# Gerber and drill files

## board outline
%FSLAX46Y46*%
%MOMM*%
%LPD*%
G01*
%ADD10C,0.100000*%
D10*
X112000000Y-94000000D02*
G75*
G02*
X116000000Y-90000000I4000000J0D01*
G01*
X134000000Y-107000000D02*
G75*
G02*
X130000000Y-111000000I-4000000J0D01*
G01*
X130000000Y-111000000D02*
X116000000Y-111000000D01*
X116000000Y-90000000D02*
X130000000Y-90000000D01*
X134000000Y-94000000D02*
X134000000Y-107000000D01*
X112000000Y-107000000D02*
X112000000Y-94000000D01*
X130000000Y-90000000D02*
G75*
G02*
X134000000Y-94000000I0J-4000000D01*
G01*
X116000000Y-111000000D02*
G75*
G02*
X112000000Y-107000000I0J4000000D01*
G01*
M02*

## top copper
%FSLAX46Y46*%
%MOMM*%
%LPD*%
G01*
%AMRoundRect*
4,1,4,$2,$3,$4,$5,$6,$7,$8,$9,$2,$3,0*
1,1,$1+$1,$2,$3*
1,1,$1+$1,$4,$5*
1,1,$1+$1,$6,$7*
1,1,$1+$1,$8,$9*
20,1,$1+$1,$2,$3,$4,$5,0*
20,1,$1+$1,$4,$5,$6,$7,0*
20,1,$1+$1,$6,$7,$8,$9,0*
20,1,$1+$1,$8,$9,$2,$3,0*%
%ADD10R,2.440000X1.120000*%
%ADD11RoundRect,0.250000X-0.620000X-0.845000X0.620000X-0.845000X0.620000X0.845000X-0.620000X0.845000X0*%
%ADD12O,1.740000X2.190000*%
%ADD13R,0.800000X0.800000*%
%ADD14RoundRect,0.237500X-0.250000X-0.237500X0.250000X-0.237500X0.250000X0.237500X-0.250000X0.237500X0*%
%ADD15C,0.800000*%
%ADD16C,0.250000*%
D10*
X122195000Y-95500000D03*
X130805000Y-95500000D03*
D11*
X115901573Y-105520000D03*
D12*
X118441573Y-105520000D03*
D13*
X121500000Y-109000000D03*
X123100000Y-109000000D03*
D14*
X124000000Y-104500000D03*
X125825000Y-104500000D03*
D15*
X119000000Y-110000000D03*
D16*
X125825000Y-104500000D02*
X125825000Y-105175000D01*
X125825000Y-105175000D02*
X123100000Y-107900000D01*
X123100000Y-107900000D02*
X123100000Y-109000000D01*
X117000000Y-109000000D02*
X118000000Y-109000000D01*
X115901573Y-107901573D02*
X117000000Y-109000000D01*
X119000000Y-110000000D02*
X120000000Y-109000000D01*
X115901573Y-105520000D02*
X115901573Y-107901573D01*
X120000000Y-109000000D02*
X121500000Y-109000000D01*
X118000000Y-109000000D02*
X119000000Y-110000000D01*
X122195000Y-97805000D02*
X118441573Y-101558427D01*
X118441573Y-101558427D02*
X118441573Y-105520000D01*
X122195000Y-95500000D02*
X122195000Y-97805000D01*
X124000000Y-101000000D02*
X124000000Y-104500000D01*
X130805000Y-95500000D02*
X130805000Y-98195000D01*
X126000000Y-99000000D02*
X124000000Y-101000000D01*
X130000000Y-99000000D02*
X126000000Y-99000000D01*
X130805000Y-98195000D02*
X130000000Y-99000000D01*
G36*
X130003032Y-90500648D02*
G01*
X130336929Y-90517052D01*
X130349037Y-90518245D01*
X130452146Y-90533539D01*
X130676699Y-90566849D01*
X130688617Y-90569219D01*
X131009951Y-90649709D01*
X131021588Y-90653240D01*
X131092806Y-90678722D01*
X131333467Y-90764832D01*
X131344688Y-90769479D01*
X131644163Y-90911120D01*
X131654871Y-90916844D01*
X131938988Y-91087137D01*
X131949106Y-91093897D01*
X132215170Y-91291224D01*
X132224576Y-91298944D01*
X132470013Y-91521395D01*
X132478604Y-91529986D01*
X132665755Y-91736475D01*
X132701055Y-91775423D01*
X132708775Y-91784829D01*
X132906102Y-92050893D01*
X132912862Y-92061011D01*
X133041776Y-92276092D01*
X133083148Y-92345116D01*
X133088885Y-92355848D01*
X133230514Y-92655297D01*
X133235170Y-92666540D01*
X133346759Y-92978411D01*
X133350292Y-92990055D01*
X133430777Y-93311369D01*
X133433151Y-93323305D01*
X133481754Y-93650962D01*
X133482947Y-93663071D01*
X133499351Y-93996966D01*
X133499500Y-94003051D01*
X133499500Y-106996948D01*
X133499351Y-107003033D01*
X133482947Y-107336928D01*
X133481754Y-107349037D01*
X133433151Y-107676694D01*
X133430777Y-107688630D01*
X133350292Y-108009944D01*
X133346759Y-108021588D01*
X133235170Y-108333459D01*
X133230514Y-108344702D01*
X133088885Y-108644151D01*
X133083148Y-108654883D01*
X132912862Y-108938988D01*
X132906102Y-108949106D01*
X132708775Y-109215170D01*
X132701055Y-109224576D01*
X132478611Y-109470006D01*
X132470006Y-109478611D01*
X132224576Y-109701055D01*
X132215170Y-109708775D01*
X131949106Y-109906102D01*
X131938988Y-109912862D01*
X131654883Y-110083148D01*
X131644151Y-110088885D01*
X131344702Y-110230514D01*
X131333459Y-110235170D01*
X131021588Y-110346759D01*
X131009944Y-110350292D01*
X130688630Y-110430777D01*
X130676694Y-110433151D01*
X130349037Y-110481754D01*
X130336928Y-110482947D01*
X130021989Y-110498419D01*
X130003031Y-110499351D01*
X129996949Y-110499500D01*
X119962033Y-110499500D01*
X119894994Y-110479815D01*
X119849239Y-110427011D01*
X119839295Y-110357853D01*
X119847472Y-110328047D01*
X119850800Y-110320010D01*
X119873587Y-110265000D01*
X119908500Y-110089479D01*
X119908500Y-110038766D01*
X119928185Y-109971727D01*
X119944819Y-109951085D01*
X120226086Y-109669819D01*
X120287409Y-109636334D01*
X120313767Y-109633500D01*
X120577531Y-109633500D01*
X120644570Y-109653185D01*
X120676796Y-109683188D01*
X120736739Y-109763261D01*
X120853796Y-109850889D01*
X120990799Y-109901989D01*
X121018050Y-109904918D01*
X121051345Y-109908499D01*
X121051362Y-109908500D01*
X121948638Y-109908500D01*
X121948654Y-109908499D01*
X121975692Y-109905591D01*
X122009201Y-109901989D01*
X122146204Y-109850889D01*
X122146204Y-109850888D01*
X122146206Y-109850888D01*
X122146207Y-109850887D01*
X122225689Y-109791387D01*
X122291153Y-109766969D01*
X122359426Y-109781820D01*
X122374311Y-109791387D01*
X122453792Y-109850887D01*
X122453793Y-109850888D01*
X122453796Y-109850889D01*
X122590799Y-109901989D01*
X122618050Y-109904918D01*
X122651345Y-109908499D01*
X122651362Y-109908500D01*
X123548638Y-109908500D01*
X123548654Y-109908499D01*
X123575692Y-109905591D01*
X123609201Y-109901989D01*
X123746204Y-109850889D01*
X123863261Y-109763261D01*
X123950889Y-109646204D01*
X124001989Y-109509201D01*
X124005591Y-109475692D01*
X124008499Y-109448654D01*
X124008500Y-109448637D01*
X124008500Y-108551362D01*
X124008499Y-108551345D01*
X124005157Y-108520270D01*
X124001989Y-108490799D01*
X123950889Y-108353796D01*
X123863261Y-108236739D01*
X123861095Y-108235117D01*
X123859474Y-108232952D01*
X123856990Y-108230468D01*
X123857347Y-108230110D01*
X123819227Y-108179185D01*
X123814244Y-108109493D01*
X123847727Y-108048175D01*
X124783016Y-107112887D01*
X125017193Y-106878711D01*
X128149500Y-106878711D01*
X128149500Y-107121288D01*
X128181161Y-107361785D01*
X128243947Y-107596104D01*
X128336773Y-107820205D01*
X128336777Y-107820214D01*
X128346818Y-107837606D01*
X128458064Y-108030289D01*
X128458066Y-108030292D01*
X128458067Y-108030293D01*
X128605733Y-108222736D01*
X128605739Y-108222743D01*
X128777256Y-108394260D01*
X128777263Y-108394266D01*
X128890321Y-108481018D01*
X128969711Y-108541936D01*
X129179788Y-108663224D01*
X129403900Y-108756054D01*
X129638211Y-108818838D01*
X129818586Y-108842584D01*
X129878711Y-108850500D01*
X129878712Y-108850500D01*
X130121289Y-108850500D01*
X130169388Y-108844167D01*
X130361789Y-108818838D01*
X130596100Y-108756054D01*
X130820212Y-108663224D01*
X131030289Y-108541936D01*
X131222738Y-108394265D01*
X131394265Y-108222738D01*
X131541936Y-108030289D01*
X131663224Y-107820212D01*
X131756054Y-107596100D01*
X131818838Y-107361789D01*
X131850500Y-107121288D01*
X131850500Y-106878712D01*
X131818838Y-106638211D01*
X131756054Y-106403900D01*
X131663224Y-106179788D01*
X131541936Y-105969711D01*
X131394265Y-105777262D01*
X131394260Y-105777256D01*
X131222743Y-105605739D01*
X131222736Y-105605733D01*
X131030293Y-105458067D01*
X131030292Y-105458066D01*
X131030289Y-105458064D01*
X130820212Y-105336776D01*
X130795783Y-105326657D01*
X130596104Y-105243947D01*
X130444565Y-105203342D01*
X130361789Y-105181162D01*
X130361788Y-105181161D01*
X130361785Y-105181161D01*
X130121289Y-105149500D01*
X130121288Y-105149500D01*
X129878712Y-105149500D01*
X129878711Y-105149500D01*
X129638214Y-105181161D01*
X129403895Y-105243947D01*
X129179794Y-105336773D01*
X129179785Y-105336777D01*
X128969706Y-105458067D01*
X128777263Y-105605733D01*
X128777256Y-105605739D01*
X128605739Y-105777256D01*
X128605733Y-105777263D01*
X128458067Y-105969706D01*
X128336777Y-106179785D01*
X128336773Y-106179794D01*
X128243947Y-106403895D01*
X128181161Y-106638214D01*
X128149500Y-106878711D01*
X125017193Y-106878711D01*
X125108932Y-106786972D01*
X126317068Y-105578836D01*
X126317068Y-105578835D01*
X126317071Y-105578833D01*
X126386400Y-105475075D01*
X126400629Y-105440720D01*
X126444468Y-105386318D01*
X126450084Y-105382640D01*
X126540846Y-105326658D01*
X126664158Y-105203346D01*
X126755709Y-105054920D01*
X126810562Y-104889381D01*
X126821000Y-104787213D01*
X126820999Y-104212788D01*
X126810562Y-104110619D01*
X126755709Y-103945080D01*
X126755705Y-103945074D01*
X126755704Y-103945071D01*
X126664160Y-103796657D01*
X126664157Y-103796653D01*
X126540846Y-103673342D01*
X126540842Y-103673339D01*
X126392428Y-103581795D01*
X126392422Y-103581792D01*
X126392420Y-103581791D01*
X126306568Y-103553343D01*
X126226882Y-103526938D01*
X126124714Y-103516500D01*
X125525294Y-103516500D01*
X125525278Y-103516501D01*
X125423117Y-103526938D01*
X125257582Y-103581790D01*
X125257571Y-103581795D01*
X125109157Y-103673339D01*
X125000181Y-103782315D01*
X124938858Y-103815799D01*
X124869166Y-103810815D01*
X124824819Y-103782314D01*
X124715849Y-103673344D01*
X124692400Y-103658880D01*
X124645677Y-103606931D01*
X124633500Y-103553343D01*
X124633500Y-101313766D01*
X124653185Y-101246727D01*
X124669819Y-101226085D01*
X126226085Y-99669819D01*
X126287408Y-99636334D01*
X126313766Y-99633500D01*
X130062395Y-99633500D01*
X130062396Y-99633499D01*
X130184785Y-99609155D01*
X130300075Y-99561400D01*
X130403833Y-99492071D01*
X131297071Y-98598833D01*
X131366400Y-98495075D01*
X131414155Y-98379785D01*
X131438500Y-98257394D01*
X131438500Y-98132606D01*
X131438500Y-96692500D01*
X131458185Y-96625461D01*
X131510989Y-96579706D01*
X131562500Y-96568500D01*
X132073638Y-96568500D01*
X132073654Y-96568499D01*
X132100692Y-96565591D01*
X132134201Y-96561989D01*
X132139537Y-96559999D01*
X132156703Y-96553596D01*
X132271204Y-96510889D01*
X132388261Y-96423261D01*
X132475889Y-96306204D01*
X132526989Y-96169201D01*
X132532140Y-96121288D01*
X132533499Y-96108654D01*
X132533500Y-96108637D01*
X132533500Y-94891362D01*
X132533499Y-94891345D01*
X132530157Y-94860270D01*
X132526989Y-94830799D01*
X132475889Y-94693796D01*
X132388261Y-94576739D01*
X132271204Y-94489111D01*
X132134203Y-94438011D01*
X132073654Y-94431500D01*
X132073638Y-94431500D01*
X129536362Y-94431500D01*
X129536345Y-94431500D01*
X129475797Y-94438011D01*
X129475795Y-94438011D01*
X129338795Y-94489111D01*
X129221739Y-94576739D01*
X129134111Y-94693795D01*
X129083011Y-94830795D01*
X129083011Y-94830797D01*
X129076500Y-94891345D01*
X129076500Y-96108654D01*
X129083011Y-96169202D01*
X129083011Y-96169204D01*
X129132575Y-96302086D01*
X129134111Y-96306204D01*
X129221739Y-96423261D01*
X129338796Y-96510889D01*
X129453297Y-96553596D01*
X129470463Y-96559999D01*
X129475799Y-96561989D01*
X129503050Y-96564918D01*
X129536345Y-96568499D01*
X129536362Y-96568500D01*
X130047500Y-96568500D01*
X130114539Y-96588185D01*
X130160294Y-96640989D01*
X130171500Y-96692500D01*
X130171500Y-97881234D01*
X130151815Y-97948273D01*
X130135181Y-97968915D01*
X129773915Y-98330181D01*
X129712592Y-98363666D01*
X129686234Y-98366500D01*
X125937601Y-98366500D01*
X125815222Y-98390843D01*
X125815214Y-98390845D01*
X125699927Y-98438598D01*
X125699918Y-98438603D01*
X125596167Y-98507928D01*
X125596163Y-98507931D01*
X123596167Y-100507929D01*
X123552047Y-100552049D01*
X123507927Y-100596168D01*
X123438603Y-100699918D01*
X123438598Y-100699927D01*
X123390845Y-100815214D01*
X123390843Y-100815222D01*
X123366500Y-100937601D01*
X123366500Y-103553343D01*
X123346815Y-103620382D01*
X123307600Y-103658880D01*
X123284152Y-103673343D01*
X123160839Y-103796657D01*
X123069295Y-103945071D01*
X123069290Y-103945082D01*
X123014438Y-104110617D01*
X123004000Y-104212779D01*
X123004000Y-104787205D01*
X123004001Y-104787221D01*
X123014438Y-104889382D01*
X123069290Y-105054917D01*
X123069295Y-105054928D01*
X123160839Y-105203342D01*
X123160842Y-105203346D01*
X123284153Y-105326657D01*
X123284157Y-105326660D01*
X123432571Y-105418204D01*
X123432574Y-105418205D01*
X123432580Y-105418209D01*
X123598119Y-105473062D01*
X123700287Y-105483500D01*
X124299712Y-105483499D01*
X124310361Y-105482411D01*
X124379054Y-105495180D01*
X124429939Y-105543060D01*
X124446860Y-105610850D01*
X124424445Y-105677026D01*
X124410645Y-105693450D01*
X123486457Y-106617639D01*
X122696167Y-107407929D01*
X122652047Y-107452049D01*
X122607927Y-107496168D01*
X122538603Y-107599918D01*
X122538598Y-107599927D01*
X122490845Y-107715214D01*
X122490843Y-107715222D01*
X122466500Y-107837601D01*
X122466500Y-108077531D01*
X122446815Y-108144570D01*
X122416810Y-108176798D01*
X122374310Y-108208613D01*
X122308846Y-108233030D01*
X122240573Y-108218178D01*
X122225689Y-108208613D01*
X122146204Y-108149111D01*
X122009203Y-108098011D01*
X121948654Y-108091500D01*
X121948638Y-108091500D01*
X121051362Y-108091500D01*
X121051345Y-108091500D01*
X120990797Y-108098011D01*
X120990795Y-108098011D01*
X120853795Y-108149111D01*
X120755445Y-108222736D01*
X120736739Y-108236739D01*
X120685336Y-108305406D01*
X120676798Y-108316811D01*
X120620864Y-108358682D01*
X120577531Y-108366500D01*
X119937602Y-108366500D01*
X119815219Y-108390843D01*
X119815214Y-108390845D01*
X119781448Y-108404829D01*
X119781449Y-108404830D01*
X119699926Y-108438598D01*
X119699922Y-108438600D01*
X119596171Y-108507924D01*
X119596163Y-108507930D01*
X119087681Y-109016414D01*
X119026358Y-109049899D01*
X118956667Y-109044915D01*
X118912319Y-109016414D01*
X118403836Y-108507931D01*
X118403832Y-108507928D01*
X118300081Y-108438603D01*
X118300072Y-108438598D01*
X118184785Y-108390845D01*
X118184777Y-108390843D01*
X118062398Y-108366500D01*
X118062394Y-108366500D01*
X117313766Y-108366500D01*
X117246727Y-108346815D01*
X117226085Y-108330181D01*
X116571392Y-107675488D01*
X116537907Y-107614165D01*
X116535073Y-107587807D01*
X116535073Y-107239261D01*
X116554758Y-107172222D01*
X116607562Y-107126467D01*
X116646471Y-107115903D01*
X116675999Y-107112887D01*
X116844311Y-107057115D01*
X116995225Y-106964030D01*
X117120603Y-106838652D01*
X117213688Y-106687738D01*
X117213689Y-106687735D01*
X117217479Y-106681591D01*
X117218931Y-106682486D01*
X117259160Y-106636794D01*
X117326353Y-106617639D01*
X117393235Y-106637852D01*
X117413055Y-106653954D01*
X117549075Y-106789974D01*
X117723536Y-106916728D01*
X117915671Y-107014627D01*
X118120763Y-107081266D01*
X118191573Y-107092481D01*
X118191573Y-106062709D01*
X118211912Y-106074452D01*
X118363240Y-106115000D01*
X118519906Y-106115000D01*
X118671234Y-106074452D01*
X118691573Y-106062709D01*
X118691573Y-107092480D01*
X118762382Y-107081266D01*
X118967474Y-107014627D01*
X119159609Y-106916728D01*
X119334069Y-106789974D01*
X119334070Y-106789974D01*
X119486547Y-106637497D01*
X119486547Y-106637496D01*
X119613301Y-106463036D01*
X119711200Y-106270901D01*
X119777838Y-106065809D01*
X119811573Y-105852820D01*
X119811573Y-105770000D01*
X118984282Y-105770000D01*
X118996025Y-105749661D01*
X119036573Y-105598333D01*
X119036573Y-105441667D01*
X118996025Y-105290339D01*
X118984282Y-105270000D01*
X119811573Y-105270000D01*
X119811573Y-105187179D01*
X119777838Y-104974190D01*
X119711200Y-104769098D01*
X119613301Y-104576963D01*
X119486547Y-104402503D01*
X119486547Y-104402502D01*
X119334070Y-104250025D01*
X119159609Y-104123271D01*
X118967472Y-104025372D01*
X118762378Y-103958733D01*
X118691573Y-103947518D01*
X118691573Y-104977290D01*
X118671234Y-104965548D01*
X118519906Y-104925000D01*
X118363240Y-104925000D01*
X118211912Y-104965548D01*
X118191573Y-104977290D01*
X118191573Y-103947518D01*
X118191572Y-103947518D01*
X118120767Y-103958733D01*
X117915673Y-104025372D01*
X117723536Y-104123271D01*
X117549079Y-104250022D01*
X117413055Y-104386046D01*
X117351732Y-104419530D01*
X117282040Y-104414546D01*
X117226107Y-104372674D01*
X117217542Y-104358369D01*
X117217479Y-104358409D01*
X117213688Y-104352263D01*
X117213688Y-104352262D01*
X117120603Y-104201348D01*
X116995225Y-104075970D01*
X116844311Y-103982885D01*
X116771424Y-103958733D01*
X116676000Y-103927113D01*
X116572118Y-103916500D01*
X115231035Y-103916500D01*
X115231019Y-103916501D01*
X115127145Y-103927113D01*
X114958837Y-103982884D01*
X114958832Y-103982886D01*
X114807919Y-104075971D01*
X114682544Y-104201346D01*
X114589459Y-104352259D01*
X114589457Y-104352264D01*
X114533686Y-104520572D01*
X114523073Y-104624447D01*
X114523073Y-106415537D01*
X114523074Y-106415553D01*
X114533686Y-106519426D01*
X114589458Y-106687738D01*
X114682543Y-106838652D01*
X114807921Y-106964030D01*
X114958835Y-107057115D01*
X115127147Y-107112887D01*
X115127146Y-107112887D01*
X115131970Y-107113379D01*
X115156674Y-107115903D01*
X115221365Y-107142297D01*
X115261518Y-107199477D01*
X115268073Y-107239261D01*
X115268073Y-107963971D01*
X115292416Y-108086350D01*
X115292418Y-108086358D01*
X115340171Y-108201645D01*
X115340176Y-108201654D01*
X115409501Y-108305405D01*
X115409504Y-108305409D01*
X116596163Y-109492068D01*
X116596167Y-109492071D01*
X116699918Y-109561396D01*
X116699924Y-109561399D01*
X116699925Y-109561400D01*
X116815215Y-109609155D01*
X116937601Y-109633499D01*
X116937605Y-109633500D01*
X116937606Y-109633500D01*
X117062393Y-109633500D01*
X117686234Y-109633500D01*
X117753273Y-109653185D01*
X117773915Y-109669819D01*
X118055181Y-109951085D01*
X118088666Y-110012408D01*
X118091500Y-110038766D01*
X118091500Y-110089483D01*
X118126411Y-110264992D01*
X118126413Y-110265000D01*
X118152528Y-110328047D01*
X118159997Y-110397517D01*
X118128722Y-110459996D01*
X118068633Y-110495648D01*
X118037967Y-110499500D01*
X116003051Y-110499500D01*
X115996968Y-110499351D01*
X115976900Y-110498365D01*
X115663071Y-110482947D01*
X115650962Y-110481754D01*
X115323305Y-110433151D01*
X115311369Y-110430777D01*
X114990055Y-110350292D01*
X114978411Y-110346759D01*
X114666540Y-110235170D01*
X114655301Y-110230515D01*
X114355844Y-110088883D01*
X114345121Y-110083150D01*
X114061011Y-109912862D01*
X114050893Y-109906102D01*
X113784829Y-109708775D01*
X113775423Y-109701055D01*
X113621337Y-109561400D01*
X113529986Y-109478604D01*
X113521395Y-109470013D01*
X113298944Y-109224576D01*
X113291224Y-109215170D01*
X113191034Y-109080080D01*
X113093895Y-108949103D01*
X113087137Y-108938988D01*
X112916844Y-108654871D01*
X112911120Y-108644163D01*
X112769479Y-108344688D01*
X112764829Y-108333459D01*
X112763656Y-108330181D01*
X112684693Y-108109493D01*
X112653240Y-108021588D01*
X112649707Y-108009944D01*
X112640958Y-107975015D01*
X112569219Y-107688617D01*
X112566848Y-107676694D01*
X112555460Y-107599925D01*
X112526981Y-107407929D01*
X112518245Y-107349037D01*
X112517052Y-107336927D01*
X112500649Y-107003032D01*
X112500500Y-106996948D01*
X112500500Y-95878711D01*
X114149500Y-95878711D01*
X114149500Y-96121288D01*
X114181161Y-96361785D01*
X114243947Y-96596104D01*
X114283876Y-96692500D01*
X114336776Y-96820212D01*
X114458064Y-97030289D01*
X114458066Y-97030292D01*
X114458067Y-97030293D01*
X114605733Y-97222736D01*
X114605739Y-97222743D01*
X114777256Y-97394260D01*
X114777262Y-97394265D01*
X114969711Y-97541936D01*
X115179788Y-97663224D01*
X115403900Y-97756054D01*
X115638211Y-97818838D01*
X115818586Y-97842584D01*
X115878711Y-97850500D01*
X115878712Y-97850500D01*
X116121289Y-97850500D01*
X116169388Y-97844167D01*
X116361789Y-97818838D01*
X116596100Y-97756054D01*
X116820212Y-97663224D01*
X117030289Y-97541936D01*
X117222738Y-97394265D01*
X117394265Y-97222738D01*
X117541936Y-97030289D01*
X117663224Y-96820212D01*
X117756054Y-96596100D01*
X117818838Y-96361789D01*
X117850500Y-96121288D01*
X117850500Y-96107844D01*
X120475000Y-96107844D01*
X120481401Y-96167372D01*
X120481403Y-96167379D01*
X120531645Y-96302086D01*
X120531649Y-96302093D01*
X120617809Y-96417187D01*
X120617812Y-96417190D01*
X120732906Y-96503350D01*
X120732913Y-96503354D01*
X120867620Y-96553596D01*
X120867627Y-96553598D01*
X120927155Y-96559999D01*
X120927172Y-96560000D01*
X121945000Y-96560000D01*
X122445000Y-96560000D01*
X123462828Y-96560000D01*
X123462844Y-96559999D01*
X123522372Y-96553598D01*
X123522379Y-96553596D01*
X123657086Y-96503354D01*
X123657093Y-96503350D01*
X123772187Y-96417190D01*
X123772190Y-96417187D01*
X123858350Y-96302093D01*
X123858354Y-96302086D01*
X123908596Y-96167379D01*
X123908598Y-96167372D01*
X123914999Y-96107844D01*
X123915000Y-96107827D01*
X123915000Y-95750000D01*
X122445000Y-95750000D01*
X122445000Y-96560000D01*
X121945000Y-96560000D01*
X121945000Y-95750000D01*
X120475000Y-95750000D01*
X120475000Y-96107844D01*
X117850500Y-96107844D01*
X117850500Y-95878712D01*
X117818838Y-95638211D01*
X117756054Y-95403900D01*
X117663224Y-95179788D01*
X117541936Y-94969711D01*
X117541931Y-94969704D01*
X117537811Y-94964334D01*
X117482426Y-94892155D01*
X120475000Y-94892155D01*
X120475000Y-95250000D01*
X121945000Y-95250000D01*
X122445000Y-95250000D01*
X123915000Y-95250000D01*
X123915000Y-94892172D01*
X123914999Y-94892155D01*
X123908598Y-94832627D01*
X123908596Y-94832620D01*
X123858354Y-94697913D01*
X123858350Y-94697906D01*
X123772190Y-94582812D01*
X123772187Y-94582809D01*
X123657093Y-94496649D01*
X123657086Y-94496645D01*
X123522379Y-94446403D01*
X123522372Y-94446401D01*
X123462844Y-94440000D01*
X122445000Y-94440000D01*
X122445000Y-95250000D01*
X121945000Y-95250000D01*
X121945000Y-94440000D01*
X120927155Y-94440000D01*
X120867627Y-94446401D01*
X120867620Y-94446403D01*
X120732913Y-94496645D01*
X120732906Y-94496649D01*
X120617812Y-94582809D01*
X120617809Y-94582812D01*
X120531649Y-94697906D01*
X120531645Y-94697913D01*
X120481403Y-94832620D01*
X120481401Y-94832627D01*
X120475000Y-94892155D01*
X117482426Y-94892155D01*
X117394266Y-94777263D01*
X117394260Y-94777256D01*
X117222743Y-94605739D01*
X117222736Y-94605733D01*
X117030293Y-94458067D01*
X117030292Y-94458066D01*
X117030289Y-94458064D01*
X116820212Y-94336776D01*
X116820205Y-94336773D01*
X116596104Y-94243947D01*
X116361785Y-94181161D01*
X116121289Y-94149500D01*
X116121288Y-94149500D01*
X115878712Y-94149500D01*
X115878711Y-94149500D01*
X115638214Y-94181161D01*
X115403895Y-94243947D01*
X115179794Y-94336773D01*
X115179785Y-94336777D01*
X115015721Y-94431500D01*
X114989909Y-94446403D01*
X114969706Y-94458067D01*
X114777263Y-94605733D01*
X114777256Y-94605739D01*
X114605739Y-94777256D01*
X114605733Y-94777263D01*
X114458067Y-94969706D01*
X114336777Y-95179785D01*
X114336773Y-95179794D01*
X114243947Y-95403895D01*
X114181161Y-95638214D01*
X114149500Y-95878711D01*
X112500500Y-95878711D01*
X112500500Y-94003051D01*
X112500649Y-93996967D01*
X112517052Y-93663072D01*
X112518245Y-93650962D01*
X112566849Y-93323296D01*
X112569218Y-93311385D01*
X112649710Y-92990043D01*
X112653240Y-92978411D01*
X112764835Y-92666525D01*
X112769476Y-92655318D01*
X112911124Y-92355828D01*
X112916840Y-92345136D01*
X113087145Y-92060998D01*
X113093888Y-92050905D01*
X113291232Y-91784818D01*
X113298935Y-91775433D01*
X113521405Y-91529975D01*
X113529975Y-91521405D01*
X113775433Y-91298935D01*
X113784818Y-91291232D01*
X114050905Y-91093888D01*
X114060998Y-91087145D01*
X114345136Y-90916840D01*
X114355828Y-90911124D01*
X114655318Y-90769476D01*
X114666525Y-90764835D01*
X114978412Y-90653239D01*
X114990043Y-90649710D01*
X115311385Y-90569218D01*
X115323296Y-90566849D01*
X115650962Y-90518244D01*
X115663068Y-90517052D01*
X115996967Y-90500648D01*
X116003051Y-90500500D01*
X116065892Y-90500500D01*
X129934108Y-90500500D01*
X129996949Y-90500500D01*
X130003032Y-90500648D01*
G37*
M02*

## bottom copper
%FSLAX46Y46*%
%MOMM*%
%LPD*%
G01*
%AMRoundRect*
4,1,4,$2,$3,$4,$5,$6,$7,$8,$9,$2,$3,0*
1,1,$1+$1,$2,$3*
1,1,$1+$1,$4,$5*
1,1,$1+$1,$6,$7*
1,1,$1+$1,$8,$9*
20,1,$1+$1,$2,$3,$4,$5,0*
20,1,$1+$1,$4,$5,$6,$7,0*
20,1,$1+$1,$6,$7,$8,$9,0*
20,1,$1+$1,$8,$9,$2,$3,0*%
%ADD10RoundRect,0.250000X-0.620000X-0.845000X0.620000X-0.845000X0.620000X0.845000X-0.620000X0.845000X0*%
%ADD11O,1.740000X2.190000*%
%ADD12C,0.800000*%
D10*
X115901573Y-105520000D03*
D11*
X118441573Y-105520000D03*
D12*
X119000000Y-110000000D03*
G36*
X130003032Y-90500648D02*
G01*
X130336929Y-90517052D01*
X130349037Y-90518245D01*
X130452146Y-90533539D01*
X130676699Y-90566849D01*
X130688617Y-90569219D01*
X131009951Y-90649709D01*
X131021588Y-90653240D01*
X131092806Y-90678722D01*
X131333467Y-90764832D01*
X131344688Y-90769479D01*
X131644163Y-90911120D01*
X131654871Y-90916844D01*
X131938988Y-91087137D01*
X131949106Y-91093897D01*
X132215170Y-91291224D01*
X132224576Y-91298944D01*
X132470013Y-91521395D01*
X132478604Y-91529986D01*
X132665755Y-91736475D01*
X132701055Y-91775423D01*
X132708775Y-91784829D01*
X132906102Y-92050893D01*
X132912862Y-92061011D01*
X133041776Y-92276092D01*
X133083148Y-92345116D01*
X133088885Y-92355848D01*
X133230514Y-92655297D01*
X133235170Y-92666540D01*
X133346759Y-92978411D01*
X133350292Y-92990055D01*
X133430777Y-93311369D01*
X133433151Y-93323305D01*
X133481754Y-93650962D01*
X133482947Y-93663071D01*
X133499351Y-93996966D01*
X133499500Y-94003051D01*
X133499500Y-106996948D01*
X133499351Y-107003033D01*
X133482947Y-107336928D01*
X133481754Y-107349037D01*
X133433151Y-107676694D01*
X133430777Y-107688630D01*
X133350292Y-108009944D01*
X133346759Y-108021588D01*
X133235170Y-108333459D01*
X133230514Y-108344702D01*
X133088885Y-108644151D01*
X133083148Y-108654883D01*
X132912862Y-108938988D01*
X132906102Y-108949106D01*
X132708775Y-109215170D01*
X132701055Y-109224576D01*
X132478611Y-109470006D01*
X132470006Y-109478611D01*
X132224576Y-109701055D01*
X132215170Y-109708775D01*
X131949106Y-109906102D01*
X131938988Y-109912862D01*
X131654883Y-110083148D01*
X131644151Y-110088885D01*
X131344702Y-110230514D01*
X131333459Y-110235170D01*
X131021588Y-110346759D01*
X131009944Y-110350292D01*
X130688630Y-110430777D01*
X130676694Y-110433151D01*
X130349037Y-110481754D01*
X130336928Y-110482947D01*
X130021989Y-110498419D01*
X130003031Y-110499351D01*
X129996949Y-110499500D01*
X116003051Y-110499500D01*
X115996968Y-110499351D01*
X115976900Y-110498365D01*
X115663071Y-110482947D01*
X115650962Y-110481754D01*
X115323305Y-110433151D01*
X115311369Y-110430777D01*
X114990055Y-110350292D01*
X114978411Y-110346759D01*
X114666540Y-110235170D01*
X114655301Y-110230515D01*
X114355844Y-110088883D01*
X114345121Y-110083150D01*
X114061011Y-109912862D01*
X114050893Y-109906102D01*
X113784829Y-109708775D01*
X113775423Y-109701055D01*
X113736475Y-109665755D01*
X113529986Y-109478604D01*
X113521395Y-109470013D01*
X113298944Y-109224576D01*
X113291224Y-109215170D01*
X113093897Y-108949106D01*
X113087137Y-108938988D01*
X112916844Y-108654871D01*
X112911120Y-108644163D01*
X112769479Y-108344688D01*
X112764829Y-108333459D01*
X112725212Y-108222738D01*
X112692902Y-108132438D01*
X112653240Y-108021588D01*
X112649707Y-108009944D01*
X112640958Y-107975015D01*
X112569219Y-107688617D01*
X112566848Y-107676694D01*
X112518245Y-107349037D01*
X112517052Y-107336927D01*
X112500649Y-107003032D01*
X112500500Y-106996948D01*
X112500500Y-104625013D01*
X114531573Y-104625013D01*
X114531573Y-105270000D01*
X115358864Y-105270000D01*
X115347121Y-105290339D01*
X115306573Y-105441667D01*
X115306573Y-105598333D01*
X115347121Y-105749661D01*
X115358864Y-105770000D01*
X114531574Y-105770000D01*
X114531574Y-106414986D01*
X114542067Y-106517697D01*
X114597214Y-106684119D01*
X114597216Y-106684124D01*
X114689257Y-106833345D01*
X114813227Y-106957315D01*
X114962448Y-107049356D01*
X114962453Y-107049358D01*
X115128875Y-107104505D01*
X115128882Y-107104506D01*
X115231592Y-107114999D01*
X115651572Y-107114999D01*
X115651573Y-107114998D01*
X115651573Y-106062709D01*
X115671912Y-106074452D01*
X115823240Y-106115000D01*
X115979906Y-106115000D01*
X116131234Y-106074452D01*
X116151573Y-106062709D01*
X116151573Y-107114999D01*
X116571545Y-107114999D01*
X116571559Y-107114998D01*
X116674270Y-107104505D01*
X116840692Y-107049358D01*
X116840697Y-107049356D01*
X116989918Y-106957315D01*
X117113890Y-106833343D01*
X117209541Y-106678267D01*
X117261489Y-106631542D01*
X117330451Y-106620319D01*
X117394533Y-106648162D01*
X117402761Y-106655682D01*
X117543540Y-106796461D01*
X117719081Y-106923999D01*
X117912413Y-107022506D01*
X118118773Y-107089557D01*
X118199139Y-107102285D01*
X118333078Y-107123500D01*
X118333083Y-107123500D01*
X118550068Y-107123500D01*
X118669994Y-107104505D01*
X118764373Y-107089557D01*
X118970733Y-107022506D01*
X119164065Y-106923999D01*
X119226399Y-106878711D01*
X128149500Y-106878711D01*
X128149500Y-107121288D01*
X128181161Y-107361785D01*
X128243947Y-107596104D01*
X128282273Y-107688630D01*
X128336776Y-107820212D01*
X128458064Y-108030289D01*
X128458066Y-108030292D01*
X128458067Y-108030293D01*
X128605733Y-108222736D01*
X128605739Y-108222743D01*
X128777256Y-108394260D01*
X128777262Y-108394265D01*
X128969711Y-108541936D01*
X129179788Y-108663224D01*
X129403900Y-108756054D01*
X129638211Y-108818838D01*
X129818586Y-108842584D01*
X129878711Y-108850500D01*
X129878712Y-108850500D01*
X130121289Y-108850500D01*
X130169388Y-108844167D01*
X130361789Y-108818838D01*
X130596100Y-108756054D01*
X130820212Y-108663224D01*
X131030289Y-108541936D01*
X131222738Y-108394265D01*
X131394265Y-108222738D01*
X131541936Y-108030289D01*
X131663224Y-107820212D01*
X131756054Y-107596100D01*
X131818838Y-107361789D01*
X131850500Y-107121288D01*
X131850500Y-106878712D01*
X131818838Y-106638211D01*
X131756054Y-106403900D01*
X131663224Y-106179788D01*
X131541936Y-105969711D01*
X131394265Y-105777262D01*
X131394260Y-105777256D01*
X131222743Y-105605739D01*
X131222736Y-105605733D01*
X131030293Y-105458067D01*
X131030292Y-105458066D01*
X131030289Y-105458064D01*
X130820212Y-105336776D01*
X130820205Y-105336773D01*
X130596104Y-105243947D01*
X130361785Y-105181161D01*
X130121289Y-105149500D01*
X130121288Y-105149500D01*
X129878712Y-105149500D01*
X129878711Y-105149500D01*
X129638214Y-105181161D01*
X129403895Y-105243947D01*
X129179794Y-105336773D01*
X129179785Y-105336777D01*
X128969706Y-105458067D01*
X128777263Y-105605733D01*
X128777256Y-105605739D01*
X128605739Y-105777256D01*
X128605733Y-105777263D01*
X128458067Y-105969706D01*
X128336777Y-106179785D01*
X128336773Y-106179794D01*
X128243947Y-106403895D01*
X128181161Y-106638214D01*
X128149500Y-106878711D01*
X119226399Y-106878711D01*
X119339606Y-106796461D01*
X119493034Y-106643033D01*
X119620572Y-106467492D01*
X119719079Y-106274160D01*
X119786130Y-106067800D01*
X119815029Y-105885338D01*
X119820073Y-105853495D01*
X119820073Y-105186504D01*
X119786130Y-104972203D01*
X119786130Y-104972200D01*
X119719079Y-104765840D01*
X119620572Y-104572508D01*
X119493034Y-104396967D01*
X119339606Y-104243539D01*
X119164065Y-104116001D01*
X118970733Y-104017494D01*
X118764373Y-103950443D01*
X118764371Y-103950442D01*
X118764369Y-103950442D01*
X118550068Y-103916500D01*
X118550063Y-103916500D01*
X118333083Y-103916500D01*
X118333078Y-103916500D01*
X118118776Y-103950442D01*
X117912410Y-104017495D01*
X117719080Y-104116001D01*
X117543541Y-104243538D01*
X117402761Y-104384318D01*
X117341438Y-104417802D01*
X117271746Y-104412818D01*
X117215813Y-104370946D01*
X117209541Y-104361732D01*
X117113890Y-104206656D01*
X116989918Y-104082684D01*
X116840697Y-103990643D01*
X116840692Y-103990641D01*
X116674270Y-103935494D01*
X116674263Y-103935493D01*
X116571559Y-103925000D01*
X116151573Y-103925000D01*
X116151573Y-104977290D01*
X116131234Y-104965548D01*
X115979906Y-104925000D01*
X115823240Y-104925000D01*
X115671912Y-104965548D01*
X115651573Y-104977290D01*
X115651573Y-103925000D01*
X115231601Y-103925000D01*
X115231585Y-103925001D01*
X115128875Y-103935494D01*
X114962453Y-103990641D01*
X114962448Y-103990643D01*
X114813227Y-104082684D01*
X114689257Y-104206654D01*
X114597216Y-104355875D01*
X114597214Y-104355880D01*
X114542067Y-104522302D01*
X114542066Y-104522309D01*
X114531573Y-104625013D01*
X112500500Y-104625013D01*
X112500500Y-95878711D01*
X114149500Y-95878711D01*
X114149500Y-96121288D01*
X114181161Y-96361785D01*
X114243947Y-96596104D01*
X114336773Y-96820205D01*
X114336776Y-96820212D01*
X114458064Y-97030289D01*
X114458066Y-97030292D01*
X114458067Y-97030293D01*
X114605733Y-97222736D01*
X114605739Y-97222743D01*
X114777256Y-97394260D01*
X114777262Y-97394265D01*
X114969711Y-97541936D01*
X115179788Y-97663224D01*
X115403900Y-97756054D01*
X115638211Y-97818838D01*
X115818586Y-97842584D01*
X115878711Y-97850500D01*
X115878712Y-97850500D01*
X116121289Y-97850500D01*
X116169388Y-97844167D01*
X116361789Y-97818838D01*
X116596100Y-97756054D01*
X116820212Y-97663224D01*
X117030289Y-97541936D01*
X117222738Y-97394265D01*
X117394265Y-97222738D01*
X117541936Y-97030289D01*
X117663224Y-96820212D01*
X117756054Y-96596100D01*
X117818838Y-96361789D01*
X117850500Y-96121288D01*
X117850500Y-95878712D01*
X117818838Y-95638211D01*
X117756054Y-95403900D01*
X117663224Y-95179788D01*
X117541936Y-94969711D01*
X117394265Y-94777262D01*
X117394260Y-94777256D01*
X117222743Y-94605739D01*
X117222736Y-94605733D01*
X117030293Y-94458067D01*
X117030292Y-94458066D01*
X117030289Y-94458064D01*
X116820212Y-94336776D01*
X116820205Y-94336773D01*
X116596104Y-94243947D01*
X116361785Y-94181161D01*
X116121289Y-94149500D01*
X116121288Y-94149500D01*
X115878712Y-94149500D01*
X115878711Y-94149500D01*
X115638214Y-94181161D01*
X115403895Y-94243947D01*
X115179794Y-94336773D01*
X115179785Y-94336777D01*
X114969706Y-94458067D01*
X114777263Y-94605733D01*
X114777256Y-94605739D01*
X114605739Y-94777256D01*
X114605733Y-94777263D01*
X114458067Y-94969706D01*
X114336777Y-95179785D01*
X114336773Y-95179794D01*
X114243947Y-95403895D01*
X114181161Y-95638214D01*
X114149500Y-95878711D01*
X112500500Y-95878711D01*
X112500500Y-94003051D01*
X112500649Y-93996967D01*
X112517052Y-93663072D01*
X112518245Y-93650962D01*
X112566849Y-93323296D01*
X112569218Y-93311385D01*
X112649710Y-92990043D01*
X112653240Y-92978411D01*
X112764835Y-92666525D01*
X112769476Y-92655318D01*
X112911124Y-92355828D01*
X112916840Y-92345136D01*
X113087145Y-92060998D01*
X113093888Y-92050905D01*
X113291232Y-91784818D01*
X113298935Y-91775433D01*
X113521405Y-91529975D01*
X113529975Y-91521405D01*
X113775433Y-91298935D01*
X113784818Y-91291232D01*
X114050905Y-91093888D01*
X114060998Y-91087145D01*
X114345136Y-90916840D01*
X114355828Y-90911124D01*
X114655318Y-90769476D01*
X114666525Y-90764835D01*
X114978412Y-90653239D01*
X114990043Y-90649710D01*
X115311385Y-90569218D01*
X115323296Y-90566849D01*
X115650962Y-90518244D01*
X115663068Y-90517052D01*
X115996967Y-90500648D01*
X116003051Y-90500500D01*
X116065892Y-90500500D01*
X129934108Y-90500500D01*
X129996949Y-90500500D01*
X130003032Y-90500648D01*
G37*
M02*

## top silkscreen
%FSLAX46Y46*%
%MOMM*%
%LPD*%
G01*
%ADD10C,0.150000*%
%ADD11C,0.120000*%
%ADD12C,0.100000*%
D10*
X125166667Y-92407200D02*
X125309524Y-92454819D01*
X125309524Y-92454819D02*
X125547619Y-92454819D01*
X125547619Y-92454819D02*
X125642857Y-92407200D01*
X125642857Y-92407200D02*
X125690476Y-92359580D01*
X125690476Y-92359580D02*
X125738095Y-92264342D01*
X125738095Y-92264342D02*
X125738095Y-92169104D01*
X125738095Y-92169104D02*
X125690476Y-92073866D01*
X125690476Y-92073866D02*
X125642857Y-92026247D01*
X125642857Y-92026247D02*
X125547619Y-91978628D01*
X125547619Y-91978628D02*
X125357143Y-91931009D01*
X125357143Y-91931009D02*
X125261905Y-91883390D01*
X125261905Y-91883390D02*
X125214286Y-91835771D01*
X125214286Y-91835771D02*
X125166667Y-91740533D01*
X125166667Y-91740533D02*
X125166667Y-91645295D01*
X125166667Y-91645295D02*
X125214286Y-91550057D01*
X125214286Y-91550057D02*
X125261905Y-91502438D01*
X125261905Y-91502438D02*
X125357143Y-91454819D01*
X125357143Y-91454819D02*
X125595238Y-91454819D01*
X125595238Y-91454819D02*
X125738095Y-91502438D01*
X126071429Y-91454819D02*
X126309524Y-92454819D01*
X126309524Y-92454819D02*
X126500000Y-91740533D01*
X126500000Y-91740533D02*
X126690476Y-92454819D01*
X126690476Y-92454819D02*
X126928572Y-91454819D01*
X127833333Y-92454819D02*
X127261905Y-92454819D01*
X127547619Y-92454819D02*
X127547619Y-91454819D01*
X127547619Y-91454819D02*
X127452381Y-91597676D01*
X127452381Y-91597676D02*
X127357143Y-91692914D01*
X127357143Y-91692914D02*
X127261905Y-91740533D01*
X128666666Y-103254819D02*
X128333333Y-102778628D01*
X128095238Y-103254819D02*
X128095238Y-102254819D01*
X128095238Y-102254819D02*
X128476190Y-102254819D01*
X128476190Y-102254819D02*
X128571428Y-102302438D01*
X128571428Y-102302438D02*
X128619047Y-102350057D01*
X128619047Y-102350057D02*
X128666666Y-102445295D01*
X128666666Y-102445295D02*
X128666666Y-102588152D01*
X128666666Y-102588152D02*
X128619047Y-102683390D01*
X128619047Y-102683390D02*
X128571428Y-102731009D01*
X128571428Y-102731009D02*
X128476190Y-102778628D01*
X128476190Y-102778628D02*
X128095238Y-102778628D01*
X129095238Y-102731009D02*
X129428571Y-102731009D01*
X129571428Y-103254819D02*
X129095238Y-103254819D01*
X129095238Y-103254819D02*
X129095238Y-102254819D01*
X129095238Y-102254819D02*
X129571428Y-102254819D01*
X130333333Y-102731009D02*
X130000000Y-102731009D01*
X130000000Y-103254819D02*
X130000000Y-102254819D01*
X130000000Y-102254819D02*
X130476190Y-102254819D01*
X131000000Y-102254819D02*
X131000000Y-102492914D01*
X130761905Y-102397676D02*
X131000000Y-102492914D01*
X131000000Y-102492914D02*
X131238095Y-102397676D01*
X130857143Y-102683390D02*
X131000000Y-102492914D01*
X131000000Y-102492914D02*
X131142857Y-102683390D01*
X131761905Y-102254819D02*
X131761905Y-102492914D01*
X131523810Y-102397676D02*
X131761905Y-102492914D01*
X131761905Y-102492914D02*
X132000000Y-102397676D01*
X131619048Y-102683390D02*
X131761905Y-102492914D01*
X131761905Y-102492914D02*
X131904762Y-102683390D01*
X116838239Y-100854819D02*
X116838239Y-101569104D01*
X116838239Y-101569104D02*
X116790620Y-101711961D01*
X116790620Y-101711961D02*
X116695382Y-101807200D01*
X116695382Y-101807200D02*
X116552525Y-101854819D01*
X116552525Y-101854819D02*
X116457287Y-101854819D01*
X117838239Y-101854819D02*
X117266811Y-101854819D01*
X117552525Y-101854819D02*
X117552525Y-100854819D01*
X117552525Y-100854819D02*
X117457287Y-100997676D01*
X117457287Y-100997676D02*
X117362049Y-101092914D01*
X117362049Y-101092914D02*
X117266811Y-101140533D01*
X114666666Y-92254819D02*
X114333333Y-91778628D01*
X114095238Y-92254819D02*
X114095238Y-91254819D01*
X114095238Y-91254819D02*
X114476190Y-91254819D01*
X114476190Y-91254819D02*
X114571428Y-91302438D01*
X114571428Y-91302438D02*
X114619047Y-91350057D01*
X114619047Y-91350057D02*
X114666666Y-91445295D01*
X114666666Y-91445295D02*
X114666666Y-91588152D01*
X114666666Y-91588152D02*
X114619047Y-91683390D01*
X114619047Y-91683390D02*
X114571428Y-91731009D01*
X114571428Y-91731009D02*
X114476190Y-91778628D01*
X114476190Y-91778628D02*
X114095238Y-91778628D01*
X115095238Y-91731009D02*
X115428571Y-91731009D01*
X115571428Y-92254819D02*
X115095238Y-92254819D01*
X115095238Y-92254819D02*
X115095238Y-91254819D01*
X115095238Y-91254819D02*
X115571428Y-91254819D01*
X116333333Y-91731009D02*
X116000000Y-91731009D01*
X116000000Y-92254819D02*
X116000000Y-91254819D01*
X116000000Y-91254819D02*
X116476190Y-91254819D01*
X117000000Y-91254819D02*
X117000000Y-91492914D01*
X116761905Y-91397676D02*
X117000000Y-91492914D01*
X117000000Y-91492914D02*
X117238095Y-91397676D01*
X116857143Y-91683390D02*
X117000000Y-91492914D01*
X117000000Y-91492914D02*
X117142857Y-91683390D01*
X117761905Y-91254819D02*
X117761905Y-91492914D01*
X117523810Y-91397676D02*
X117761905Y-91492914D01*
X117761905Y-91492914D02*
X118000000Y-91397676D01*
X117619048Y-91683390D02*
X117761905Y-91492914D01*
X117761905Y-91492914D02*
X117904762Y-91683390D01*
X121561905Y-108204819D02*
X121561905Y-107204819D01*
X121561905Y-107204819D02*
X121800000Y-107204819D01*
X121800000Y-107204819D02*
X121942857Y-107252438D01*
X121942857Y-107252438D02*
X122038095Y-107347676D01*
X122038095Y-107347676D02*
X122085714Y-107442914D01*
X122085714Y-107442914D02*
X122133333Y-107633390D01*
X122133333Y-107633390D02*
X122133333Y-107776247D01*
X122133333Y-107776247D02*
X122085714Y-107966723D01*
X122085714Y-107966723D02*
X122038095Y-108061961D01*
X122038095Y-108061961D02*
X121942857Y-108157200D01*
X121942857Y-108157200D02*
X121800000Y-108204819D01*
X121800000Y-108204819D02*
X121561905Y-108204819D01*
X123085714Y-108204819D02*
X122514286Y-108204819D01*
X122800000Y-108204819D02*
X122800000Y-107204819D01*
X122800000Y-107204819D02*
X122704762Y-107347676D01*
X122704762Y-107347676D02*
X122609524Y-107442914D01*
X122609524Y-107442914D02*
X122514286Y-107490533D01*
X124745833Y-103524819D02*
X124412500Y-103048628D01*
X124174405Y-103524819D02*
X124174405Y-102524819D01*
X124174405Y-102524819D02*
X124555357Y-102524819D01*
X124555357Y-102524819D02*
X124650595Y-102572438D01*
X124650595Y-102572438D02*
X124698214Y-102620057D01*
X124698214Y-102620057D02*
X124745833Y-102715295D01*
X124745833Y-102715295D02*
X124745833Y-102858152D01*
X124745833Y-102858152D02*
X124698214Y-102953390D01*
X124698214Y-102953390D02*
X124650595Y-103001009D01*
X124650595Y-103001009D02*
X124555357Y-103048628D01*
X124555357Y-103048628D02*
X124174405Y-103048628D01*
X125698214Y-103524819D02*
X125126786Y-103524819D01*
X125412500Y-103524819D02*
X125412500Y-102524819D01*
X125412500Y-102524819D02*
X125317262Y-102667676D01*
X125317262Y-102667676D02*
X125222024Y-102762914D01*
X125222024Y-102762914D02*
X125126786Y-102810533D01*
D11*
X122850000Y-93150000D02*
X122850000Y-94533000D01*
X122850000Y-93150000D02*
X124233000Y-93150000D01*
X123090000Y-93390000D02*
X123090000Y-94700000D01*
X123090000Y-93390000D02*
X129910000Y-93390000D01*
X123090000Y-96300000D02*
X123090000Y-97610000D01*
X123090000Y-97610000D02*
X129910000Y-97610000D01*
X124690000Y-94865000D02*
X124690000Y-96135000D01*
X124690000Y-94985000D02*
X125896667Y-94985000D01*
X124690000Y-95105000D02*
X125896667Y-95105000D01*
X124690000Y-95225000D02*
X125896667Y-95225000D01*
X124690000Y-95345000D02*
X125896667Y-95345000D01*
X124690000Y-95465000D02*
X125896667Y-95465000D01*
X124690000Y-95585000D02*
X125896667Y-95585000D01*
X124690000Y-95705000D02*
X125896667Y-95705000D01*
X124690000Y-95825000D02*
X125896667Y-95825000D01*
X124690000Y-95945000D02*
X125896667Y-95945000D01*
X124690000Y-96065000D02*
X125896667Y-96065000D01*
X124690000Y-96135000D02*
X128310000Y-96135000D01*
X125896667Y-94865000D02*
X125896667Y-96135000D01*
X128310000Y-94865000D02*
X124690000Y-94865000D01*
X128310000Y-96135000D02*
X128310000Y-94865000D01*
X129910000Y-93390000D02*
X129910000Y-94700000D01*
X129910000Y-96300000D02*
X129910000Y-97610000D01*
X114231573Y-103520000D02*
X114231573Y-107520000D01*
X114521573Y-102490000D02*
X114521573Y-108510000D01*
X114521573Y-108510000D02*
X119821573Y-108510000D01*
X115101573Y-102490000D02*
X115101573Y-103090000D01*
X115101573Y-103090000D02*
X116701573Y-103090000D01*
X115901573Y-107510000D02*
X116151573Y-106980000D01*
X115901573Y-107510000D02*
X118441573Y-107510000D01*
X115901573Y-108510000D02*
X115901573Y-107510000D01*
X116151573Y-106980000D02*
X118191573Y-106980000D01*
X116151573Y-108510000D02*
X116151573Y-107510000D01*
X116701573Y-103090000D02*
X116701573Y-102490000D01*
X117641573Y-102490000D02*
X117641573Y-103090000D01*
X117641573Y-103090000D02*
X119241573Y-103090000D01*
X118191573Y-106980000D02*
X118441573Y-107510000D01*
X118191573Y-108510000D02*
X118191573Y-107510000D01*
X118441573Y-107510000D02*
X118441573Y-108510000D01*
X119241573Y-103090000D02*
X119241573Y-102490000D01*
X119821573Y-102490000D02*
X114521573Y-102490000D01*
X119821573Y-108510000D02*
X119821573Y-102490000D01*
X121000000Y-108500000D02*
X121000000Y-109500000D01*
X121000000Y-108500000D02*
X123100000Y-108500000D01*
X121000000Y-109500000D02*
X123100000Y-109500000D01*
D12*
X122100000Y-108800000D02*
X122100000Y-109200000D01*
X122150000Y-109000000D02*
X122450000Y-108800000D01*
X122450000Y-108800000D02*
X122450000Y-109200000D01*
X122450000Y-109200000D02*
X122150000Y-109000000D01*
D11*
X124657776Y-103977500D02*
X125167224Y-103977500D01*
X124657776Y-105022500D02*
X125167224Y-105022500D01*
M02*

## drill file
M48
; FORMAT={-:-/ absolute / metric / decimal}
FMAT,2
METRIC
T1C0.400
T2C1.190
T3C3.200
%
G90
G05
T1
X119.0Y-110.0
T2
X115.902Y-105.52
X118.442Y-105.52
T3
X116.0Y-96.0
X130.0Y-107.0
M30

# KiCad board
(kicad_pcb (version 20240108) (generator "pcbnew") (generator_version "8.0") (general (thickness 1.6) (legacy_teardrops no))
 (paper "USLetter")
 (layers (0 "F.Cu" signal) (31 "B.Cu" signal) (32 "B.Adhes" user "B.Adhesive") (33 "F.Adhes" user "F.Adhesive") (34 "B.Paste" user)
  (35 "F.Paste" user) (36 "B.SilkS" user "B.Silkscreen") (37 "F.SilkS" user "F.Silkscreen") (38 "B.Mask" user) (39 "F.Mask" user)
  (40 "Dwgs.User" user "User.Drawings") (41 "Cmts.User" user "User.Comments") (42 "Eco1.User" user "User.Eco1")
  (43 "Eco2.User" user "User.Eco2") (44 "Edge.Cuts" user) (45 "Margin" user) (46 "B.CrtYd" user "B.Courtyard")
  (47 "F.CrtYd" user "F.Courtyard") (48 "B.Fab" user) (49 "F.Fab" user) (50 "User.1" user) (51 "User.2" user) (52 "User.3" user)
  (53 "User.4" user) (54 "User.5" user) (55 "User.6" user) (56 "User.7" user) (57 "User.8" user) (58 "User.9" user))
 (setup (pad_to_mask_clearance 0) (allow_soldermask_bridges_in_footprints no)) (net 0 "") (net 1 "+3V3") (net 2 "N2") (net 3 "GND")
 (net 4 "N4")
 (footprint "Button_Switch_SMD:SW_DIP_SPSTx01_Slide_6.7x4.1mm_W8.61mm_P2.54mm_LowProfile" (layer "F.Cu") (at 126.5 95.5)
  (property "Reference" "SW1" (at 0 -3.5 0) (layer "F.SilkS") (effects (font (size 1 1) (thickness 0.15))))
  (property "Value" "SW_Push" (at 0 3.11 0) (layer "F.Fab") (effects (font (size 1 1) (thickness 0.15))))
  (fp_line (start -3.65 -2.35) (end -3.65 -0.967) (stroke (width 0.12) (type solid)) (layer "F.SilkS"))
  (fp_line (start -3.65 -2.35) (end -2.267 -2.35) (stroke (width 0.12) (type solid)) (layer "F.SilkS"))
  (fp_line (start -3.41 -2.11) (end -3.41 -0.8) (stroke (width 0.12) (type solid)) (layer "F.SilkS"))
  (fp_line (start -3.41 -2.11) (end 3.41 -2.11) (stroke (width 0.12) (type solid)) (layer "F.SilkS"))
  (fp_line (start -3.41 0.8) (end -3.41 2.11) (stroke (width 0.12) (type solid)) (layer "F.SilkS"))
  (fp_line (start -3.41 2.11) (end 3.41 2.11) (stroke (width 0.12) (type solid)) (layer "F.SilkS"))
  (fp_line (start -1.81 -0.635) (end -1.81 0.635) (stroke (width 0.12) (type solid)) (layer "F.SilkS"))
  (fp_line (start -1.81 -0.515) (end -0.603333 -0.515) (stroke (width 0.12) (type solid)) (layer "F.SilkS"))
  (fp_line (start -1.81 -0.395) (end -0.603333 -0.395) (stroke (width 0.12) (type solid)) (layer "F.SilkS"))
  (fp_line (start -1.81 -0.275) (end -0.603333 -0.275) (stroke (width 0.12) (type solid)) (layer "F.SilkS"))
  (fp_line (start -1.81 -0.155) (end -0.603333 -0.155) (stroke (width 0.12) (type solid)) (layer "F.SilkS"))
  (fp_line (start -1.81 -0.035) (end -0.603333 -0.035) (stroke (width 0.12) (type solid)) (layer "F.SilkS"))
  (fp_line (start -1.81 0.085) (end -0.603333 0.085) (stroke (width 0.12) (type solid)) (layer "F.SilkS"))
  (fp_line (start -1.81 0.205) (end -0.603333 0.205) (stroke (width 0.12) (type solid)) (layer "F.SilkS"))
  (fp_line (start -1.81 0.325) (end -0.603333 0.325) (stroke (width 0.12) (type solid)) (layer "F.SilkS"))
  (fp_line (start -1.81 0.445) (end -0.603333 0.445) (stroke (width 0.12) (type solid)) (layer "F.SilkS"))
  (fp_line (start -1.81 0.565) (end -0.603333 0.565) (stroke (width 0.12) (type solid)) (layer "F.SilkS"))
  (fp_line (start -1.81 0.635) (end 1.81 0.635) (stroke (width 0.12) (type solid)) (layer "F.SilkS"))
  (fp_line (start -0.603333 -0.635) (end -0.603333 0.635) (stroke (width 0.12) (type solid)) (layer "F.SilkS"))
  (fp_line (start 1.81 -0.635) (end -1.81 -0.635) (stroke (width 0.12) (type solid)) (layer "F.SilkS"))
  (fp_line (start 1.81 0.635) (end 1.81 -0.635) (stroke (width 0.12) (type solid)) (layer "F.SilkS"))
  (fp_line (start 3.41 -2.11) (end 3.41 -0.8) (stroke (width 0.12) (type solid)) (layer "F.SilkS"))
  (fp_line (start 3.41 0.8) (end 3.41 2.11) (stroke (width 0.12) (type solid)) (layer "F.SilkS"))
  (pad "1" smd rect (at -4.305 0) (size 2.44 1.12) (layers "F.Cu" "F.Paste" "F.Mask") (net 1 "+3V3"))
  (pad "2" smd rect (at 4.305 0) (size 2.44 1.12) (layers "F.Cu" "F.Paste" "F.Mask") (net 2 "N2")))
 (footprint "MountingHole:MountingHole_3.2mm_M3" (layer "F.Cu") (at 130 107)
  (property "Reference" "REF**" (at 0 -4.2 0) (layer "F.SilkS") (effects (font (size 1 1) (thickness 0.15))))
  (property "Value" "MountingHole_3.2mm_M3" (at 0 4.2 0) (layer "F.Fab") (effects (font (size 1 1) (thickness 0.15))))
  (pad "" np_thru_hole circle (at 0 0) (size 3.2 3.2) (drill 3.2) (layers "*.Cu" "*.Mask")))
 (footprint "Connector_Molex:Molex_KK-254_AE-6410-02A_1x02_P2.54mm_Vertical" (layer "F.Cu") (at 115.901573 105.52)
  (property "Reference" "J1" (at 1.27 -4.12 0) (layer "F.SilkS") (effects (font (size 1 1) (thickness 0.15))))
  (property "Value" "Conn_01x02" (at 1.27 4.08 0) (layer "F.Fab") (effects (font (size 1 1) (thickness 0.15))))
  (fp_line (start -1.67 -2) (end -1.67 2) (stroke (width 0.12) (type solid)) (layer "F.SilkS"))
  (fp_line (start -1.38 -3.03) (end -1.38 2.99) (stroke (width 0.12) (type solid)) (layer "F.SilkS"))
  (fp_line (start -1.38 2.99) (end 3.92 2.99) (stroke (width 0.12) (type solid)) (layer "F.SilkS"))
  (fp_line (start -0.8 -3.03) (end -0.8 -2.43) (stroke (width 0.12) (type solid)) (layer "F.SilkS"))
  (fp_line (start -0.8 -2.43) (end 0.8 -2.43) (stroke (width 0.12) (type solid)) (layer "F.SilkS"))
  (fp_line (start 0 1.99) (end 0.25 1.46) (stroke (width 0.12) (type solid)) (layer "F.SilkS"))
  (fp_line (start 0 1.99) (end 2.54 1.99) (stroke (width 0.12) (type solid)) (layer "F.SilkS"))
  (fp_line (start 0 2.99) (end 0 1.99) (stroke (width 0.12) (type solid)) (layer "F.SilkS"))
  (fp_line (start 0.25 1.46) (end 2.29 1.46) (stroke (width 0.12) (type solid)) (layer "F.SilkS"))
  (fp_line (start 0.25 2.99) (end 0.25 1.99) (stroke (width 0.12) (type solid)) (layer "F.SilkS"))
  (fp_line (start 0.8 -2.43) (end 0.8 -3.03) (stroke (width 0.12) (type solid)) (layer "F.SilkS"))
  (fp_line (start 1.74 -3.03) (end 1.74 -2.43) (stroke (width 0.12) (type solid)) (layer "F.SilkS"))
  (fp_line (start 1.74 -2.43) (end 3.34 -2.43) (stroke (width 0.12) (type solid)) (layer "F.SilkS"))
  (fp_line (start 2.29 1.46) (end 2.54 1.99) (stroke (width 0.12) (type solid)) (layer "F.SilkS"))
  (fp_line (start 2.29 2.99) (end 2.29 1.99) (stroke (width 0.12) (type solid)) (layer "F.SilkS"))
  (fp_line (start 2.54 1.99) (end 2.54 2.99) (stroke (width 0.12) (type solid)) (layer "F.SilkS"))
  (fp_line (start 3.34 -2.43) (end 3.34 -3.03) (stroke (width 0.12) (type solid)) (layer "F.SilkS"))
  (fp_line (start 3.92 -3.03) (end -1.38 -3.03) (stroke (width 0.12) (type solid)) (layer "F.SilkS"))
  (fp_line (start 3.92 2.99) (end 3.92 -3.03) (stroke (width 0.12) (type solid)) (layer "F.SilkS"))
  (pad "1" thru_hole roundrect (at 0 0) (size 1.74 2.19) (drill 1.19) (layers "*.Cu" "*.Mask") (remove_unused_layers no)
   (roundrect_rratio 0.143678) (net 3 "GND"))
  (pad "2" thru_hole oval (at 2.54 0) (size 1.74 2.19) (drill 1.19) (layers "*.Cu" "*.Mask") (remove_unused_layers no) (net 1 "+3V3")))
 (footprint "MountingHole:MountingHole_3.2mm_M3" (layer "F.Cu") (at 116 96)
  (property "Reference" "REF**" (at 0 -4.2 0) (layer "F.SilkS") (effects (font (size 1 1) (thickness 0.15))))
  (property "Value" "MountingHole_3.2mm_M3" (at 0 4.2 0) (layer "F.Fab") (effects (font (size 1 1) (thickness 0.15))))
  (pad "" np_thru_hole circle (at 0 0) (size 3.2 3.2) (drill 3.2) (layers "*.Cu" "*.Mask")))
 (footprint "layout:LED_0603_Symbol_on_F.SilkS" (layer "F.Cu") (at 122.3 109)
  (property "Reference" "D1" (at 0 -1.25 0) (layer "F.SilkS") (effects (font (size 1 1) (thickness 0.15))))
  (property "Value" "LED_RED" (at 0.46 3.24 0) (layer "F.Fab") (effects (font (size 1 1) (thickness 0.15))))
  (fp_line (start -1.3 -0.5) (end -1.3 0.5) (stroke (width 0.12) (type solid)) (layer "F.SilkS"))
  (fp_line (start -1.3 -0.5) (end 0.8 -0.5) (stroke (width 0.12) (type solid)) (layer "F.SilkS"))
  (fp_line (start -1.3 0.5) (end 0.8 0.5) (stroke (width 0.12) (type solid)) (layer "F.SilkS"))
  (fp_line (start -0.2 -0.2) (end -0.2 0.2) (stroke (width 0.1) (type solid)) (layer "F.SilkS"))
  (fp_line (start -0.15 0) (end 0.15 -0.2) (stroke (width 0.1) (type solid)) (layer "F.SilkS"))
  (fp_line (start 0.15 -0.2) (end 0.15 0.2) (stroke (width 0.1) (type solid)) (layer "F.SilkS"))
  (fp_line (start 0.15 0.2) (end -0.15 0) (stroke (width 0.1) (type solid)) (layer "F.SilkS"))
  (pad "1" smd rect (at -0.8 0 180) (size 0.8 0.8) (layers "F.Cu" "F.Paste" "F.Mask") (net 3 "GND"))
  (pad "2" smd rect (at 0.8 0 180) (size 0.8 0.8) (layers "F.Cu" "F.Paste" "F.Mask") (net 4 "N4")))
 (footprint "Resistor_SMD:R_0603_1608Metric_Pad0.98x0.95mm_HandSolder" (layer "F.Cu") (at 124.9125 104.5)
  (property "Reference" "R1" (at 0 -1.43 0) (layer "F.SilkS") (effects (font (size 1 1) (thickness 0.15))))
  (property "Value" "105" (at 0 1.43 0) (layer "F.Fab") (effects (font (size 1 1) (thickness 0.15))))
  (fp_line (start -0.254724 -0.5225) (end 0.254724 -0.5225) (stroke (width 0.12) (type solid)) (layer "F.SilkS"))
  (fp_line (start -0.254724 0.5225) (end 0.254724 0.5225) (stroke (width 0.12) (type solid)) (layer "F.SilkS"))
  (pad "1" smd roundrect (at -0.9125 0) (size 0.975 0.95) (layers "F.Cu" "F.Paste" "F.Mask") (roundrect_rratio 0.25) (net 2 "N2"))
  (pad "2" smd roundrect (at 0.9125 0) (size 0.975 0.95) (layers "F.Cu" "F.Paste" "F.Mask") (roundrect_rratio 0.25) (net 4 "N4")))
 (gr_arc (start 112 94) (mid 113.171573 91.171573) (end 116 90) (stroke (width 0.1) (type default)) (layer "Edge.Cuts"))
 (gr_arc (start 134 107) (mid 132.828427 109.828427) (end 130 111) (stroke (width 0.1) (type default)) (layer "Edge.Cuts"))
 (gr_line (start 130 111) (end 116 111) (stroke (width 0.1) (type default)) (layer "Edge.Cuts"))
 (gr_line (start 116 90) (end 130 90) (stroke (width 0.1) (type default)) (layer "Edge.Cuts"))
 (gr_line (start 134 94) (end 134 107) (stroke (width 0.1) (type default)) (layer "Edge.Cuts"))
 (gr_line (start 112 107) (end 112 94) (stroke (width 0.1) (type default)) (layer "Edge.Cuts"))
 (gr_arc (start 130 90) (mid 132.828427 91.171573) (end 134 94) (stroke (width 0.1) (type default)) (layer "Edge.Cuts"))
 (gr_arc (start 116 111) (mid 113.171573 109.828427) (end 112 107) (stroke (width 0.1) (type default)) (layer "Edge.Cuts"))
 (segment (start 125.825 104.5) (end 125.825 105.175) (width 0.25) (layer "F.Cu") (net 4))
 (segment (start 125.825 105.175) (end 123.1 107.9) (width 0.25) (layer "F.Cu") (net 4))
 (segment (start 123.1 107.9) (end 123.1 109) (width 0.25) (layer "F.Cu") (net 4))
 (segment (start 117 109) (end 118 109) (width 0.25) (layer "F.Cu") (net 3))
 (segment (start 115.901573 107.901573) (end 117 109) (width 0.25) (layer "F.Cu") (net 3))
 (segment (start 119 110) (end 120 109) (width 0.25) (layer "F.Cu") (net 3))
 (segment (start 115.901573 105.52) (end 115.901573 107.901573) (width 0.25) (layer "F.Cu") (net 3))
 (segment (start 120 109) (end 121.5 109) (width 0.25) (layer "F.Cu") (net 3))
 (segment (start 118 109) (end 119 110) (width 0.25) (layer "F.Cu") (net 3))
 (via (at 119 110) (size 0.8) (drill 0.4) (layers "F.Cu" "B.Cu") (free yes) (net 3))
 (segment (start 122.195 97.805) (end 118.441573 101.558427) (width 0.25) (layer "F.Cu") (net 1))
 (segment (start 118.441573 101.558427) (end 118.441573 105.52) (width 0.25) (layer "F.Cu") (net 1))
 (segment (start 122.195 95.5) (end 122.195 97.805) (width 0.25) (layer "F.Cu") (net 1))
 (segment (start 124 101) (end 124 104.5) (width 0.25) (layer "F.Cu") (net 2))
 (segment (start 130.805 95.5) (end 130.805 98.195) (width 0.25) (layer "F.Cu") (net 2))
 (segment (start 126 99) (end 124 101) (width 0.25) (layer "F.Cu") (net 2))
 (segment (start 130 99) (end 126 99) (width 0.25) (layer "F.Cu") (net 2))
 (segment (start 130.805 98.195) (end 130 99) (width 0.25) (layer "F.Cu") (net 2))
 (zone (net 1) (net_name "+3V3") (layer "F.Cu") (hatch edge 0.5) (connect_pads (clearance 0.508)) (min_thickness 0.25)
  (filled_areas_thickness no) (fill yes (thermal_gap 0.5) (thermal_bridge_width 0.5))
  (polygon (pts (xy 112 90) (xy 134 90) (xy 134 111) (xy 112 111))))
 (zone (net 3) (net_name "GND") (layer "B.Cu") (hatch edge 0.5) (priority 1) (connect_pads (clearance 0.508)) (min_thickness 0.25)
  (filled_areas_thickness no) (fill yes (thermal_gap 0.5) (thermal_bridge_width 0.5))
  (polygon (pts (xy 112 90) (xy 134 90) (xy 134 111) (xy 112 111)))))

